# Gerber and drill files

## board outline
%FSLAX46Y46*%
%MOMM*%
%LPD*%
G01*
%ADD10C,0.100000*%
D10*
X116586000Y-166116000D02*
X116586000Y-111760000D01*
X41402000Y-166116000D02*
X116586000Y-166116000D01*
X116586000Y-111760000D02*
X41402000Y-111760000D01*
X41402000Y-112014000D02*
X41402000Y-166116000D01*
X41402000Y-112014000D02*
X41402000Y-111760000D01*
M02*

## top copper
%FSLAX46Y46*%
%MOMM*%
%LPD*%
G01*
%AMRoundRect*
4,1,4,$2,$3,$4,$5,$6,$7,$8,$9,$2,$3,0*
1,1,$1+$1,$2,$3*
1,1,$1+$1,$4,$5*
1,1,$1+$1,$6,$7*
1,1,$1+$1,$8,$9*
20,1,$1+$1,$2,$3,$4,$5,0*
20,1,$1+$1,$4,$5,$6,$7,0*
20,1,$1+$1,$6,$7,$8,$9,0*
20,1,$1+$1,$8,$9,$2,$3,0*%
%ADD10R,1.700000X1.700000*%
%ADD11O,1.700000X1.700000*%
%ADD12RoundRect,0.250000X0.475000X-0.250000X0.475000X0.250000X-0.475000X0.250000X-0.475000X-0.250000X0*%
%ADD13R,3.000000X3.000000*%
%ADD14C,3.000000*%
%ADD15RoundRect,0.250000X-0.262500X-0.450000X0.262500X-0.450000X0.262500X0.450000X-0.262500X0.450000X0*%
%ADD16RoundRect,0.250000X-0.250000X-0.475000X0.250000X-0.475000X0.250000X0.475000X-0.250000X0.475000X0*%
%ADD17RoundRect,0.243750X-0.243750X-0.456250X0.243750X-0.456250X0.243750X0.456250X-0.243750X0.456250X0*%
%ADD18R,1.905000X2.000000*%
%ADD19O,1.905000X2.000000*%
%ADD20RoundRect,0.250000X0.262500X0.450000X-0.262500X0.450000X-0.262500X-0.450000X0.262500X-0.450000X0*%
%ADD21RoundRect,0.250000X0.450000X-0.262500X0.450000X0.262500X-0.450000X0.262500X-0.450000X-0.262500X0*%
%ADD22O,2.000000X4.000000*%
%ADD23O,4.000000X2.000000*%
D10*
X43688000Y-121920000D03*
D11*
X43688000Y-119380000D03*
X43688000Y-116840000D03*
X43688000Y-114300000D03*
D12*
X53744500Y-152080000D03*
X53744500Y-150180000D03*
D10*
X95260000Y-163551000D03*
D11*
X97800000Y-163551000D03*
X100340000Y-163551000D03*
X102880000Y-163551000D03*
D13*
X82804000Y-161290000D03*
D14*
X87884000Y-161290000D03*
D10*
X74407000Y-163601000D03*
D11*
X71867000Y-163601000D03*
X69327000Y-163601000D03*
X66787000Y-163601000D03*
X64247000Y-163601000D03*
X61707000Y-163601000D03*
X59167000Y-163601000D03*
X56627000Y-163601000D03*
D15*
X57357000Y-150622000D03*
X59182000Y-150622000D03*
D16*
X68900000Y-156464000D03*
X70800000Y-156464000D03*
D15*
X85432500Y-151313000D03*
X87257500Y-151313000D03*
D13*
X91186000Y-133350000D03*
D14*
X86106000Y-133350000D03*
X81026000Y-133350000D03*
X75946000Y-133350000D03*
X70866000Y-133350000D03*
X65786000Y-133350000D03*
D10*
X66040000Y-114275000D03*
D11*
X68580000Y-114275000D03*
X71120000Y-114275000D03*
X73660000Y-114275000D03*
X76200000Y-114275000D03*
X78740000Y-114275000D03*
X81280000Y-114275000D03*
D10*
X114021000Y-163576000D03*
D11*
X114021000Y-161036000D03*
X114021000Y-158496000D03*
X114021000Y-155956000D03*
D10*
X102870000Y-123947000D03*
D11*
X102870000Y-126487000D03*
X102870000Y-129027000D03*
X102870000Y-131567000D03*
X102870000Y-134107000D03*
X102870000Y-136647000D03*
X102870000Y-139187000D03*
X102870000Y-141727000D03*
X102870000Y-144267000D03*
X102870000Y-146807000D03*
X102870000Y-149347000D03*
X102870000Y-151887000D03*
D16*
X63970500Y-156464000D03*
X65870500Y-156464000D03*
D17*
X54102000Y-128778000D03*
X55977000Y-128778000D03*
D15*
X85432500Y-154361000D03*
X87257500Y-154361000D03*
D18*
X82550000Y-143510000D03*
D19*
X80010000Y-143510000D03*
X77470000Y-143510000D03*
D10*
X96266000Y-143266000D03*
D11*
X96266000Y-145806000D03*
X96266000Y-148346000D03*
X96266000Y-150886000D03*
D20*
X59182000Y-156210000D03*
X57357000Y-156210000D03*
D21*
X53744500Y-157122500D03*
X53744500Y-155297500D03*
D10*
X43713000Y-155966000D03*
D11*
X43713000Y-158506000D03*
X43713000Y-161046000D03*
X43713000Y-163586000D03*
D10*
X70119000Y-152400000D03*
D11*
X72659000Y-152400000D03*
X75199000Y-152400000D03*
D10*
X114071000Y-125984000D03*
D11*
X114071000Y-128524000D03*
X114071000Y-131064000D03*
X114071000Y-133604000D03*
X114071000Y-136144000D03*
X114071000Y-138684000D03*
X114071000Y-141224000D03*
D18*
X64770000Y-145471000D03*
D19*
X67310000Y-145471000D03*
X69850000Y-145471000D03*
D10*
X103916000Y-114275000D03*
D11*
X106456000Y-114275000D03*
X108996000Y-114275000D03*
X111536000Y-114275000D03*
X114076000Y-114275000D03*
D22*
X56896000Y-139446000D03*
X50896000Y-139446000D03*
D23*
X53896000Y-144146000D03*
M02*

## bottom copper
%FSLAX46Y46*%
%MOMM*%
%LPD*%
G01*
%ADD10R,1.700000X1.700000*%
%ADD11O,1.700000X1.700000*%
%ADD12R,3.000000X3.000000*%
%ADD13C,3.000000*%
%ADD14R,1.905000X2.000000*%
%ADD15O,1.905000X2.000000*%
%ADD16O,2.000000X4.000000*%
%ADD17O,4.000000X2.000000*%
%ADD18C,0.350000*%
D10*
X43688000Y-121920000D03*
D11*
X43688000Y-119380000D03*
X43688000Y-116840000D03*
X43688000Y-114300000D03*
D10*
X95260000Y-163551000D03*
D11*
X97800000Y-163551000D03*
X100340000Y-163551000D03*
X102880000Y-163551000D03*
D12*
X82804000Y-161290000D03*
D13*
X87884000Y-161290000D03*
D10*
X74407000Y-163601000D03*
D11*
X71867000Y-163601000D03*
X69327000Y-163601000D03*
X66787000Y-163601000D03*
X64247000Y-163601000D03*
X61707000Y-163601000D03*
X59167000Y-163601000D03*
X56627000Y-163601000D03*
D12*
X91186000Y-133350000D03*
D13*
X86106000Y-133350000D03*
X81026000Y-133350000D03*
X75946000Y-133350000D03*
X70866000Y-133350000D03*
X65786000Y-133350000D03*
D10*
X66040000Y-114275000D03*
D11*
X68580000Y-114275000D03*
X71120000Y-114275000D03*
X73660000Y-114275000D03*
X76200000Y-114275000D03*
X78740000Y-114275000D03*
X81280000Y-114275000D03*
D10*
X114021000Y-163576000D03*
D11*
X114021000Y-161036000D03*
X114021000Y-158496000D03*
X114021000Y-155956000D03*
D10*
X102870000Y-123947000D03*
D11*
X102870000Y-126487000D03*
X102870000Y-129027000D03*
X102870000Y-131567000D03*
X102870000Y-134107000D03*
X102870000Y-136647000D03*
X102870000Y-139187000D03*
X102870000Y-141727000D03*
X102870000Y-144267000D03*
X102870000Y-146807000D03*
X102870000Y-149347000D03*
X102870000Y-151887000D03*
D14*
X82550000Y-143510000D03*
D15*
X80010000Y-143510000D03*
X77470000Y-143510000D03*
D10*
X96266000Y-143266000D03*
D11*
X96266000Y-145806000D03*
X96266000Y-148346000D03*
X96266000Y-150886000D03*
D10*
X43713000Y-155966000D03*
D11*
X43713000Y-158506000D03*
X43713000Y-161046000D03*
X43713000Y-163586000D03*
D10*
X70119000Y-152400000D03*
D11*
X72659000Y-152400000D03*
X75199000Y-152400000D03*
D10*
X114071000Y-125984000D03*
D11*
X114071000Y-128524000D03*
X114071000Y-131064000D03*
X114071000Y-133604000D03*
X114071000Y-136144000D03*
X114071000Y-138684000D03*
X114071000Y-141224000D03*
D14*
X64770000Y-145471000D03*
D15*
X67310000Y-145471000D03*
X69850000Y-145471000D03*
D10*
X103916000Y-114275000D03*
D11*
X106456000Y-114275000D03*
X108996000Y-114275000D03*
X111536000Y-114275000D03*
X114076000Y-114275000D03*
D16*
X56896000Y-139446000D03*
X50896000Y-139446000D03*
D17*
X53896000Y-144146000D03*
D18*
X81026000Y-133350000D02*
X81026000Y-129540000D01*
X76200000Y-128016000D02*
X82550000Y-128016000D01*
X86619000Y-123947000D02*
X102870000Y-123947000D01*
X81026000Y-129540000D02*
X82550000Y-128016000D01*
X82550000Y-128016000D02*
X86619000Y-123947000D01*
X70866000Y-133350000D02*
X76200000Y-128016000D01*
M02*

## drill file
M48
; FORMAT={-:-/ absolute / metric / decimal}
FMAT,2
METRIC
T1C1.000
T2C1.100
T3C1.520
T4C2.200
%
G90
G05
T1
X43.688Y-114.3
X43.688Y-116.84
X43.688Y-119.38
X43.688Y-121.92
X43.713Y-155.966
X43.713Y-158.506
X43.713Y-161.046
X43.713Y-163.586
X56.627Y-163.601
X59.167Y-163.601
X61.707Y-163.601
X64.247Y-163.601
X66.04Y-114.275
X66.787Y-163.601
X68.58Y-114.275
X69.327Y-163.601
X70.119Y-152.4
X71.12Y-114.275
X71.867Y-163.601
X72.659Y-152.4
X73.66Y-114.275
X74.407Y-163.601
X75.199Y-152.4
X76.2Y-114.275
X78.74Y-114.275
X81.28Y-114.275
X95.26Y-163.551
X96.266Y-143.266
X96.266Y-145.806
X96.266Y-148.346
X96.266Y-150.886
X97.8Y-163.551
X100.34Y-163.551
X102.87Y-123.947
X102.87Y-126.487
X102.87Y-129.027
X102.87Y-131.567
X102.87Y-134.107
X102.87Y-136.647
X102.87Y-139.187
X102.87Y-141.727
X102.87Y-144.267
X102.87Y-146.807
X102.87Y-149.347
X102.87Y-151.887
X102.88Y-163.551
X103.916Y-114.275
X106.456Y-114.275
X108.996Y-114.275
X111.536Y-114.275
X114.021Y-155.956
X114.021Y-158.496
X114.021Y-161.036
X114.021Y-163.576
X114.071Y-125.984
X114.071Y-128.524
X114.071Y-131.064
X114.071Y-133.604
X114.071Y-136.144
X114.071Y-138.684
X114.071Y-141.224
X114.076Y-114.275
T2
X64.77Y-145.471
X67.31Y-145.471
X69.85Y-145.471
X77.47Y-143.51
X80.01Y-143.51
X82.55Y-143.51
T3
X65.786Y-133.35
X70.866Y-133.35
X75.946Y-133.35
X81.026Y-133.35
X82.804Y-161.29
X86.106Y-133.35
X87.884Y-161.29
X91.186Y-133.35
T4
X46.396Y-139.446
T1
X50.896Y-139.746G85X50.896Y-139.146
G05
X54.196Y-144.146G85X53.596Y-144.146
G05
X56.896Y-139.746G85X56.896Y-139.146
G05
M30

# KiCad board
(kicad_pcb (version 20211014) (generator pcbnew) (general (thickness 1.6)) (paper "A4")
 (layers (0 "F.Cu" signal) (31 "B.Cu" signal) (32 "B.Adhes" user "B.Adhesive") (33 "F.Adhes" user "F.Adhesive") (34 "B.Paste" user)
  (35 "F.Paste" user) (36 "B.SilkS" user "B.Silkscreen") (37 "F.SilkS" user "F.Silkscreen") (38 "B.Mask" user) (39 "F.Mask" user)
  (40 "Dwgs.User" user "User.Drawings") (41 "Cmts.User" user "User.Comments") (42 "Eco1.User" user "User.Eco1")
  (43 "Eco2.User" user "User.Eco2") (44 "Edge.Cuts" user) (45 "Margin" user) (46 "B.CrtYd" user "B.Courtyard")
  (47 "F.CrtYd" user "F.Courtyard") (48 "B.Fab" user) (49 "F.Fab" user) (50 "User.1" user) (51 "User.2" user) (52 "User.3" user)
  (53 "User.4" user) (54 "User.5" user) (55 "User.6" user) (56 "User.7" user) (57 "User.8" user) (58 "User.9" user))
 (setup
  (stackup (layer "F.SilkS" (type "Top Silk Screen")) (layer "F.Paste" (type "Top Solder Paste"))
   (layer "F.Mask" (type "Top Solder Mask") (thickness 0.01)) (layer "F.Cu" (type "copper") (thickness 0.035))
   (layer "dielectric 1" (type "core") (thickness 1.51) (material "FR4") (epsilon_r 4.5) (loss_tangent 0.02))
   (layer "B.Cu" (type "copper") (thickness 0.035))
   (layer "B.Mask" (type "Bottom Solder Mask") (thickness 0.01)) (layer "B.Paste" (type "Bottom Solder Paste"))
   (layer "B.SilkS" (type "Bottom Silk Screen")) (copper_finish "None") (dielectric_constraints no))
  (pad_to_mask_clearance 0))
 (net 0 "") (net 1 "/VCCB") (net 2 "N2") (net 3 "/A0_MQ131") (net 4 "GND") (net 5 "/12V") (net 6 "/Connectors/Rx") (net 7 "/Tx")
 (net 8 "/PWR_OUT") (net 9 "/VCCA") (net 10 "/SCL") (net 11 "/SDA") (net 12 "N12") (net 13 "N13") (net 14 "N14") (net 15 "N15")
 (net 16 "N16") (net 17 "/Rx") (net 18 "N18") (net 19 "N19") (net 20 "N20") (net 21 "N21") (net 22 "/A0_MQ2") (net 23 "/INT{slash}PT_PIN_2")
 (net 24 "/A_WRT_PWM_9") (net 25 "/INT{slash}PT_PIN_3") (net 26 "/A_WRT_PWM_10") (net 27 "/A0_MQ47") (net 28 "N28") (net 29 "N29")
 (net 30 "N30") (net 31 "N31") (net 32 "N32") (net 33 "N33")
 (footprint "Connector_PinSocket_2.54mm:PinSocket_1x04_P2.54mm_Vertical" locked (layer "F.Cu") (at 43.688 121.92 180)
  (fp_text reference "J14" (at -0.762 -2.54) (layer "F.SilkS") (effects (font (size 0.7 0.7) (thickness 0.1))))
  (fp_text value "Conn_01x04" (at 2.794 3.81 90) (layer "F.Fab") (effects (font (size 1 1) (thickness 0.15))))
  (pad "1" thru_hole rect locked (at 0 0 180) (size 1.7 1.7) (drill 1) (layers *.Cu *.Mask) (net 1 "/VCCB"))
  (pad "2" thru_hole oval locked (at 0 2.54 180) (size 1.7 1.7) (drill 1) (layers *.Cu *.Mask) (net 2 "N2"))
  (pad "3" thru_hole oval locked (at 0 5.08 180) (size 1.7 1.7) (drill 1) (layers *.Cu *.Mask) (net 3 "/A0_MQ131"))
  (pad "4" thru_hole oval locked (at 0 7.62 180) (size 1.7 1.7) (drill 1) (layers *.Cu *.Mask) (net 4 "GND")))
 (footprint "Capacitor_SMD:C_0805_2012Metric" (layer "F.Cu") (at 53.7445 151.13 90)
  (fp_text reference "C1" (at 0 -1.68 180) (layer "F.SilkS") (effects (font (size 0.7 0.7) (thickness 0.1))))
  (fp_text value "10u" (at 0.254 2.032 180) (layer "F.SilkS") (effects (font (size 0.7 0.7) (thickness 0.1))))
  (pad "1" smd roundrect locked (at -0.95 0 90) (size 1 1.45) (layers "F.Cu" "F.Paste" "F.Mask") (roundrect_rratio 0.25) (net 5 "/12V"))
  (pad "2" smd roundrect locked (at 0.95 0 90) (size 1 1.45) (layers "F.Cu" "F.Paste" "F.Mask") (roundrect_rratio 0.25) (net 4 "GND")))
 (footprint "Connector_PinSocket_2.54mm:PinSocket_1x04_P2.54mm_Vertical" (layer "F.Cu") (at 95.26 163.551 90)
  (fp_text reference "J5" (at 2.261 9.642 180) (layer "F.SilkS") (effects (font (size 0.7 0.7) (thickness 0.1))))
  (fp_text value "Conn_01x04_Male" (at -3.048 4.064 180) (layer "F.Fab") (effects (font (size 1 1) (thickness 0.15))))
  (pad "1" thru_hole rect locked (at 0 0 90) (size 1.7 1.7) (drill 1) (layers *.Cu *.Mask) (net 1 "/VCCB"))
  (pad "2" thru_hole oval locked (at 0 2.54 90) (size 1.7 1.7) (drill 1) (layers *.Cu *.Mask) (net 4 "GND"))
  (pad "3" thru_hole oval locked (at 0 5.08 90) (size 1.7 1.7) (drill 1) (layers *.Cu *.Mask) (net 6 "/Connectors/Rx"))
  (pad "4" thru_hole oval locked (at 0 7.62 90) (size 1.7 1.7) (drill 1) (layers *.Cu *.Mask) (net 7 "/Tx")))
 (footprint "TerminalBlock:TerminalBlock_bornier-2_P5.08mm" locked (layer "F.Cu") (at 82.804 161.29)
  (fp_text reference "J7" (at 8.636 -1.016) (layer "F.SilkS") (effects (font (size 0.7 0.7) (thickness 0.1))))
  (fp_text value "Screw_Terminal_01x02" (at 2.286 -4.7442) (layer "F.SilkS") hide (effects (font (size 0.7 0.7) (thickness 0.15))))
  (pad "1" thru_hole rect locked (at 0 0) (size 3 3) (drill 1.52) (layers *.Cu *.Mask) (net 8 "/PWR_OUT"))
  (pad "2" thru_hole circle locked (at 5.08 0) (size 3 3) (drill 1.52) (layers *.Cu *.Mask) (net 4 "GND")))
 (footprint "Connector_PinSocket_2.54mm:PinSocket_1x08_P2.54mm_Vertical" (layer "F.Cu") (at 74.407 163.601 -90)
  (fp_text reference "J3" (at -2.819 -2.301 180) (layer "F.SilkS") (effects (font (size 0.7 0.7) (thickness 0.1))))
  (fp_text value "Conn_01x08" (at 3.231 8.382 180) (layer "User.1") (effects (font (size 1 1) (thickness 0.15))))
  (pad "1" thru_hole rect locked (at 0 0 270) (size 1.7 1.7) (drill 1) (layers *.Cu *.Mask) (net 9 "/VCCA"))
  (pad "2" thru_hole oval locked (at 0 2.54 270) (size 1.7 1.7) (drill 1) (layers *.Cu *.Mask) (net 4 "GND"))
  (pad "3" thru_hole oval locked (at 0 5.08 270) (size 1.7 1.7) (drill 1) (layers *.Cu *.Mask) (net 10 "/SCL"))
  (pad "4" thru_hole oval locked (at 0 7.62 270) (size 1.7 1.7) (drill 1) (layers *.Cu *.Mask) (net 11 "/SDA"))
  (pad "5" thru_hole oval locked (at 0 10.16 270) (size 1.7 1.7) (drill 1) (layers *.Cu *.Mask) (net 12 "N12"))
  (pad "6" thru_hole oval locked (at 0 12.7 270) (size 1.7 1.7) (drill 1) (layers *.Cu *.Mask) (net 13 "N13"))
  (pad "7" thru_hole oval locked (at 0 15.24 270) (size 1.7 1.7) (drill 1) (layers *.Cu *.Mask) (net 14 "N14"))
  (pad "8" thru_hole oval locked (at 0 17.78 270) (size 1.7 1.7) (drill 1) (layers *.Cu *.Mask) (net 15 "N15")))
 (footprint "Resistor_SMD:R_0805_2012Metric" (layer "F.Cu") (at 58.2695 150.622)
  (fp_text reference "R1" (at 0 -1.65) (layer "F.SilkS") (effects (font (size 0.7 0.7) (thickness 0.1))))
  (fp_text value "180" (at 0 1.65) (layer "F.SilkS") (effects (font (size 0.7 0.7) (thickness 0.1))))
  (pad "1" smd roundrect locked (at -0.9125 0) (size 1.025 1.4) (layers "F.Cu" "F.Paste" "F.Mask") (roundrect_rratio 0.243902)
   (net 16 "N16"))
  (pad "2" smd roundrect locked (at 0.9125 0) (size 1.025 1.4) (layers "F.Cu" "F.Paste" "F.Mask") (roundrect_rratio 0.243902)
   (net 1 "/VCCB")))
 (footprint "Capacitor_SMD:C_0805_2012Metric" (layer "F.Cu") (at 69.85 156.464)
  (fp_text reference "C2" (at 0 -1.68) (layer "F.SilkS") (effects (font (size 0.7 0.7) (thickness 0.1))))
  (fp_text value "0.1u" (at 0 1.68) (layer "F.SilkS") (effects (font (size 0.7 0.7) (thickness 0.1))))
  (pad "1" smd roundrect locked (at -0.95 0) (size 1 1.45) (layers "F.Cu" "F.Paste" "F.Mask") (roundrect_rratio 0.25) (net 9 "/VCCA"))
  (pad "2" smd roundrect locked (at 0.95 0) (size 1 1.45) (layers "F.Cu" "F.Paste" "F.Mask") (roundrect_rratio 0.25) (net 4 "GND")))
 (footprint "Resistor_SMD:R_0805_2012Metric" (layer "F.Cu") (at 86.345 151.313)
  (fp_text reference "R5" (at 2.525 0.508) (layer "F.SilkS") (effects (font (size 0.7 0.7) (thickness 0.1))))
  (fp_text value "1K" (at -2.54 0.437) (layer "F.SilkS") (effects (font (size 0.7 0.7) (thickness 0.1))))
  (pad "1" smd roundrect locked (at -0.9125 0) (size 1.025 1.4) (layers "F.Cu" "F.Paste" "F.Mask") (roundrect_rratio 0.243902)
   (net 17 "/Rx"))
  (pad "2" smd roundrect locked (at 0.9125 0) (size 1.025 1.4) (layers "F.Cu" "F.Paste" "F.Mask") (roundrect_rratio 0.243902)
   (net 6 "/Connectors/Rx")))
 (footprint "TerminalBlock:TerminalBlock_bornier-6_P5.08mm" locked (layer "F.Cu") (at 91.186 133.35 180)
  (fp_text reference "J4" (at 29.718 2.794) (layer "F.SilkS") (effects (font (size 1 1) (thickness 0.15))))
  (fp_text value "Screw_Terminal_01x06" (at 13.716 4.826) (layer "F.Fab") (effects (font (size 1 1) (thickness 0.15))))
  (pad "1" thru_hole rect locked (at 0 0 180) (size 3 3) (drill 1.52) (layers *.Cu *.Mask) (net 4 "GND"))
  (pad "2" thru_hole circle locked (at 5.08 0 180) (size 3 3) (drill 1.52) (layers *.Cu *.Mask) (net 5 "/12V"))
  (pad "3" thru_hole circle locked (at 10.16 0 180) (size 3 3) (drill 1.52) (layers *.Cu *.Mask) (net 4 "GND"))
  (pad "4" thru_hole circle locked (at 15.24 0 180) (size 3 3) (drill 1.52) (layers *.Cu *.Mask) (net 5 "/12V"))
  (pad "5" thru_hole circle locked (at 20.32 0 180) (size 3 3) (drill 1.52) (layers *.Cu *.Mask) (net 4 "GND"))
  (pad "6" thru_hole circle locked (at 25.4 0 180) (size 3 3) (drill 1.52) (layers *.Cu *.Mask) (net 5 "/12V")))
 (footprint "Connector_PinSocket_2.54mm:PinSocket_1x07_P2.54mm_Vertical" (layer "F.Cu") (at 66.04 114.275 90)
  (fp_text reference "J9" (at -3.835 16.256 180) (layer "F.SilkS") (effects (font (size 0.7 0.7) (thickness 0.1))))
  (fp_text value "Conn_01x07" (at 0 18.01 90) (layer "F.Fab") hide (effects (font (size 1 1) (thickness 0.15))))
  (pad "1" thru_hole rect locked (at 0 0 90) (size 1.7 1.7) (drill 1) (layers *.Cu *.Mask) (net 9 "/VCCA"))
  (pad "2" thru_hole oval locked (at 0 2.54 90) (size 1.7 1.7) (drill 1) (layers *.Cu *.Mask) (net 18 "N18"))
  (pad "3" thru_hole oval locked (at 0 5.08 90) (size 1.7 1.7) (drill 1) (layers *.Cu *.Mask) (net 4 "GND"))
  (pad "4" thru_hole oval locked (at 0 7.62 90) (size 1.7 1.7) (drill 1) (layers *.Cu *.Mask) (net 10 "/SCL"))
  (pad "5" thru_hole oval locked (at 0 10.16 90) (size 1.7 1.7) (drill 1) (layers *.Cu *.Mask) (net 11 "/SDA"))
  (pad "6" thru_hole oval locked (at 0 12.7 90) (size 1.7 1.7) (drill 1) (layers *.Cu *.Mask) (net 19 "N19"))
  (pad "7" thru_hole oval locked (at 0 15.24 90) (size 1.7 1.7) (drill 1) (layers *.Cu *.Mask) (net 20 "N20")))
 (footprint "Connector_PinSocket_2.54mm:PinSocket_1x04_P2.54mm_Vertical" (layer "F.Cu") (at 114.021 163.576 180)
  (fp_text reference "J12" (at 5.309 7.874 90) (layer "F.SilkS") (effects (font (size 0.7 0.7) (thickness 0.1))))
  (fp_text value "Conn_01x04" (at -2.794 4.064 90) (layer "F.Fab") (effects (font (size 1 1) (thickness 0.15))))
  (pad "1" thru_hole rect locked (at 0 0 180) (size 1.7 1.7) (drill 1) (layers *.Cu *.Mask) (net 1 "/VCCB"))
  (pad "2" thru_hole oval locked (at 0 2.54 180) (size 1.7 1.7) (drill 1) (layers *.Cu *.Mask) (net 4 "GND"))
  (pad "3" thru_hole oval locked (at 0 5.08 180) (size 1.7 1.7) (drill 1) (layers *.Cu *.Mask) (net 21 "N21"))
  (pad "4" thru_hole oval locked (at 0 7.62 180) (size 1.7 1.7) (drill 1) (layers *.Cu *.Mask) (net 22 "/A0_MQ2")))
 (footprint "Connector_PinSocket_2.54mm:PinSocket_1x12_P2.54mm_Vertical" (layer "F.Cu") (at 102.87 123.947)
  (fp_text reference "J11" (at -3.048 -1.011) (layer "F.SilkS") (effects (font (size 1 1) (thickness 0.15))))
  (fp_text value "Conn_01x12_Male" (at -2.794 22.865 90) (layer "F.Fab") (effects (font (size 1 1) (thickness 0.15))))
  (pad "1" thru_hole rect locked (at 0 0) (size 1.7 1.7) (drill 1) (layers *.Cu *.Mask) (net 4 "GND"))
  (pad "2" thru_hole oval locked (at 0 2.54) (size 1.7 1.7) (drill 1) (layers *.Cu *.Mask) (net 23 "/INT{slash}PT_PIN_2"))
  (pad "3" thru_hole oval locked (at 0 5.08) (size 1.7 1.7) (drill 1) (layers *.Cu *.Mask) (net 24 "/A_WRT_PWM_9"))
  (pad "4" thru_hole oval locked (at 0 7.62) (size 1.7 1.7) (drill 1) (layers *.Cu *.Mask) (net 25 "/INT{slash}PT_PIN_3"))
  (pad "5" thru_hole oval locked (at 0 10.16) (size 1.7 1.7) (drill 1) (layers *.Cu *.Mask) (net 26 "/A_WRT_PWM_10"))
  (pad "6" thru_hole oval locked (at 0 12.7) (size 1.7 1.7) (drill 1) (layers *.Cu *.Mask) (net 11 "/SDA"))
  (pad "7" thru_hole oval locked (at 0 15.24) (size 1.7 1.7) (drill 1) (layers *.Cu *.Mask) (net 10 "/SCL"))
  (pad "8" thru_hole oval locked (at 0 17.78) (size 1.7 1.7) (drill 1) (layers *.Cu *.Mask) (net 22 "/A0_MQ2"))
  (pad "9" thru_hole oval locked (at 0 20.32) (size 1.7 1.7) (drill 1) (layers *.Cu *.Mask) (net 3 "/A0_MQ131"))
  (pad "10" thru_hole oval locked (at 0 22.86) (size 1.7 1.7) (drill 1) (layers *.Cu *.Mask) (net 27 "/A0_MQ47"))
  (pad "11" thru_hole oval locked (at 0 25.4) (size 1.7 1.7) (drill 1) (layers *.Cu *.Mask) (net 7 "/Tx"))
  (pad "12" thru_hole oval locked (at 0 27.94) (size 1.7 1.7) (drill 1) (layers *.Cu *.Mask) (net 17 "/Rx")))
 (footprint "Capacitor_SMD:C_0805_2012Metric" (layer "F.Cu") (at 64.9205 156.464)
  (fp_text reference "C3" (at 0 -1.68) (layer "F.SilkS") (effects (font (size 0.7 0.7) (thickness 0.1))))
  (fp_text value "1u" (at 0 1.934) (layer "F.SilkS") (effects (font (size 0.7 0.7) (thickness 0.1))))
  (pad "1" smd roundrect locked (at -0.95 0) (size 1 1.45) (layers "F.Cu" "F.Paste" "F.Mask") (roundrect_rratio 0.25) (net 1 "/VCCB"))
  (pad "2" smd roundrect locked (at 0.95 0) (size 1 1.45) (layers "F.Cu" "F.Paste" "F.Mask") (roundrect_rratio 0.25) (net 4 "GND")))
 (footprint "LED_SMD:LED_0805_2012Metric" (layer "F.Cu") (at 55.0395 128.778)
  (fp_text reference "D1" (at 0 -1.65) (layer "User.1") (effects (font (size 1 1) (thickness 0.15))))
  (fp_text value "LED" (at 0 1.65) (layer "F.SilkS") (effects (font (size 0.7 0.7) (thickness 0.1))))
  (pad "1" smd roundrect locked (at -0.9375 0) (size 0.975 1.4) (layers "F.Cu" "F.Paste" "F.Mask") (roundrect_rratio 0.25) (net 4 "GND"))
  (pad "2" smd roundrect locked (at 0.9375 0) (size 0.975 1.4) (layers "F.Cu" "F.Paste" "F.Mask") (roundrect_rratio 0.25) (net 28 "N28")))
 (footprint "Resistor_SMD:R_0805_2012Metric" (layer "F.Cu") (at 86.345 154.361)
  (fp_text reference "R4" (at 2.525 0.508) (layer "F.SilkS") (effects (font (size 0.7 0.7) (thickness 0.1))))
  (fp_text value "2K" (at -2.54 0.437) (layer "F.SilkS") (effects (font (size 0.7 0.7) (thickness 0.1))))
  (pad "1" smd roundrect locked (at -0.9125 0) (size 1.025 1.4) (layers "F.Cu" "F.Paste" "F.Mask") (roundrect_rratio 0.243902) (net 4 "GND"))
  (pad "2" smd roundrect locked (at 0.9125 0) (size 1.025 1.4) (layers "F.Cu" "F.Paste" "F.Mask") (roundrect_rratio 0.243902)
   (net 6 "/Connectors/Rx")))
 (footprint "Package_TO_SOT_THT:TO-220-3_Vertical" (layer "F.Cu") (at 82.55 143.51 180)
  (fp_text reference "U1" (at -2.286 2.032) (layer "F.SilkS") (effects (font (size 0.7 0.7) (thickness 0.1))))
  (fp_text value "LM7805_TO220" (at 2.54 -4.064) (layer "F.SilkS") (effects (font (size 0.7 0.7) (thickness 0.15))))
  (pad "1" thru_hole rect locked (at 0 0 180) (size 1.905 2) (drill 1.1) (layers *.Cu *.Mask) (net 5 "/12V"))
  (pad "2" thru_hole oval locked (at 2.54 0 180) (size 1.905 2) (drill 1.1) (layers *.Cu *.Mask) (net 4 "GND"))
  (pad "3" thru_hole oval locked (at 5.08 0 180) (size 1.905 2) (drill 1.1) (layers *.Cu *.Mask) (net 9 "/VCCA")))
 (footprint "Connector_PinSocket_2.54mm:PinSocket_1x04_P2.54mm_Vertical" (layer "F.Cu") (at 96.266 143.266)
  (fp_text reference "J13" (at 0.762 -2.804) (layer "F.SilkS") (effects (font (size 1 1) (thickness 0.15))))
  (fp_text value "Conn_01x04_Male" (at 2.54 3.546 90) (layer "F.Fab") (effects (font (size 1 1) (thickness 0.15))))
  (pad "1" thru_hole rect locked (at 0 0) (size 1.7 1.7) (drill 1) (layers *.Cu *.Mask) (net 23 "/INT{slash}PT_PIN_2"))
  (pad "2" thru_hole oval locked (at 0 2.54) (size 1.7 1.7) (drill 1) (layers *.Cu *.Mask) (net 24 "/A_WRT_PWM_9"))
  (pad "3" thru_hole oval locked (at 0 5.08) (size 1.7 1.7) (drill 1) (layers *.Cu *.Mask) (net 25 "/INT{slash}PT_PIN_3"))
  (pad "4" thru_hole oval locked (at 0 7.62) (size 1.7 1.7) (drill 1) (layers *.Cu *.Mask) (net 26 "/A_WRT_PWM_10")))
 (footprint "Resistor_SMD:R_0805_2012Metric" (layer "F.Cu") (at 58.2695 156.21 180)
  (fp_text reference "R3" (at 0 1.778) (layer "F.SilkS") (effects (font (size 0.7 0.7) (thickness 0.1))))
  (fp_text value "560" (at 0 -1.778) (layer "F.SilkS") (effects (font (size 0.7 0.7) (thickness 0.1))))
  (pad "1" smd roundrect locked (at -0.9125 0 180) (size 1.025 1.4) (layers "F.Cu" "F.Paste" "F.Mask") (roundrect_rratio 0.243902)
   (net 4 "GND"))
  (pad "2" smd roundrect locked (at 0.9125 0 180) (size 1.025 1.4) (layers "F.Cu" "F.Paste" "F.Mask") (roundrect_rratio 0.243902)
   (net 16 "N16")))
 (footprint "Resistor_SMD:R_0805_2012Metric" (layer "F.Cu") (at 53.7445 156.21 90)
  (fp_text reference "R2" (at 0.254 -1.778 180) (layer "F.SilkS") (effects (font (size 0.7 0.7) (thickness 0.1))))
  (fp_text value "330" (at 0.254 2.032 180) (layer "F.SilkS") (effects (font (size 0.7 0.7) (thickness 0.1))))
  (pad "1" smd roundrect locked (at -0.9125 0 90) (size 1.025 1.4) (layers "F.Cu" "F.Paste" "F.Mask") (roundrect_rratio 0.243902)
   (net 28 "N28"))
  (pad "2" smd roundrect locked (at 0.9125 0 90) (size 1.025 1.4) (layers "F.Cu" "F.Paste" "F.Mask") (roundrect_rratio 0.243902)
   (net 5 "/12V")))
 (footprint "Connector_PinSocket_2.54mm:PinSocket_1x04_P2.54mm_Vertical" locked (layer "F.Cu") (at 43.713 155.966)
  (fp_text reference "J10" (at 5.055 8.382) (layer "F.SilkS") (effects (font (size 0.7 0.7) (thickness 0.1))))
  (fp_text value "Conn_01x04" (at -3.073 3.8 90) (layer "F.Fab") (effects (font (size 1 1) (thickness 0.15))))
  (pad "1" thru_hole rect locked (at 0 0) (size 1.7 1.7) (drill 1) (layers *.Cu *.Mask) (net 1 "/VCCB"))
  (pad "2" thru_hole oval locked (at 0 2.54) (size 1.7 1.7) (drill 1) (layers *.Cu *.Mask) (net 4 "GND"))
  (pad "3" thru_hole oval locked (at 0 5.08) (size 1.7 1.7) (drill 1) (layers *.Cu *.Mask) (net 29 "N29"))
  (pad "4" thru_hole oval locked (at 0 7.62) (size 1.7 1.7) (drill 1) (layers *.Cu *.Mask) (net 27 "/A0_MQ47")))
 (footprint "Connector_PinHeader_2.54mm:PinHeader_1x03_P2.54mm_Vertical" (layer "F.Cu") (at 70.119 152.4 90)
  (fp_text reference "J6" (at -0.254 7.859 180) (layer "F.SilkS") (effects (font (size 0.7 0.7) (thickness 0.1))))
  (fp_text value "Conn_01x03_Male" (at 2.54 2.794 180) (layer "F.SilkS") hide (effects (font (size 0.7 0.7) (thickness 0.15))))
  (pad "1" thru_hole rect locked (at 0 0 90) (size 1.7 1.7) (drill 1) (layers *.Cu *.Mask) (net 1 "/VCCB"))
  (pad "2" thru_hole oval locked (at 0 2.54 90) (size 1.7 1.7) (drill 1) (layers *.Cu *.Mask) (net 8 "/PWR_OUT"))
  (pad "3" thru_hole oval locked (at 0 5.08 90) (size 1.7 1.7) (drill 1) (layers *.Cu *.Mask) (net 9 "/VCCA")))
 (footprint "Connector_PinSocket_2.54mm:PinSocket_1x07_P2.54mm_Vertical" (layer "F.Cu") (at 114.071 125.984)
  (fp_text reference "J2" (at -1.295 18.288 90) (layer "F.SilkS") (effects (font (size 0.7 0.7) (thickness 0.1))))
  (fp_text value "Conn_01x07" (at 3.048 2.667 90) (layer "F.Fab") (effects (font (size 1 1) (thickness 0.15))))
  (pad "1" thru_hole rect locked (at 0 0) (size 1.7 1.7) (drill 1) (layers *.Cu *.Mask) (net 9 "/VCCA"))
  (pad "2" thru_hole oval locked (at 0 2.54) (size 1.7 1.7) (drill 1) (layers *.Cu *.Mask) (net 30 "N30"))
  (pad "3" thru_hole oval locked (at 0 5.08) (size 1.7 1.7) (drill 1) (layers *.Cu *.Mask) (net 4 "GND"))
  (pad "4" thru_hole oval locked (at 0 7.62) (size 1.7 1.7) (drill 1) (layers *.Cu *.Mask) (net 10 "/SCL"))
  (pad "5" thru_hole oval locked (at 0 10.16) (size 1.7 1.7) (drill 1) (layers *.Cu *.Mask) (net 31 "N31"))
  (pad "6" thru_hole oval locked (at 0 12.7) (size 1.7 1.7) (drill 1) (layers *.Cu *.Mask) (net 11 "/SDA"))
  (pad "7" thru_hole oval locked (at 0 15.24) (size 1.7 1.7) (drill 1) (layers *.Cu *.Mask) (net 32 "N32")))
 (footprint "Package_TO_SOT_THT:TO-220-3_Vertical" (layer "F.Cu") (at 64.77 145.471)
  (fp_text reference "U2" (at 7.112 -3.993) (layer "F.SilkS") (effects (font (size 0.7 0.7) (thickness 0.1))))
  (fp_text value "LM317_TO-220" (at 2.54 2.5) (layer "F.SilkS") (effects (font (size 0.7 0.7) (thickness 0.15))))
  (pad "1" thru_hole rect locked (at 0 0) (size 1.905 2) (drill 1.1) (layers *.Cu *.Mask) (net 16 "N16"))
  (pad "2" thru_hole oval locked (at 2.54 0) (size 1.905 2) (drill 1.1) (layers *.Cu *.Mask) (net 1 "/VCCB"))
  (pad "3" thru_hole oval locked (at 5.08 0) (size 1.905 2) (drill 1.1) (layers *.Cu *.Mask) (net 5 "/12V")))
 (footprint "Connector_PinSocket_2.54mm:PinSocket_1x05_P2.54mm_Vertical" (layer "F.Cu") (at 103.916 114.275 90)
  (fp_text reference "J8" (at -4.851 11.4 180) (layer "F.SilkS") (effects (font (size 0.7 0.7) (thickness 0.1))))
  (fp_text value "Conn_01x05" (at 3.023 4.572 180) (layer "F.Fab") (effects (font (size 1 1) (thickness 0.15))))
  (pad "1" thru_hole rect locked (at 0 0 90) (size 1.7 1.7) (drill 1) (layers *.Cu *.Mask) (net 9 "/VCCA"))
  (pad "2" thru_hole oval locked (at 0 2.54 90) (size 1.7 1.7) (drill 1) (layers *.Cu *.Mask) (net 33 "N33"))
  (pad "3" thru_hole oval locked (at 0 5.08 90) (size 1.7 1.7) (drill 1) (layers *.Cu *.Mask) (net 4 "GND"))
  (pad "4" thru_hole oval locked (at 0 7.62 90) (size 1.7 1.7) (drill 1) (layers *.Cu *.Mask) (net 10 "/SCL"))
  (pad "5" thru_hole oval locked (at 0 10.16 90) (size 1.7 1.7) (drill 1) (layers *.Cu *.Mask) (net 11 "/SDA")))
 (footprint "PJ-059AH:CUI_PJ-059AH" (layer "F.Cu") (at 56.896 139.446 180)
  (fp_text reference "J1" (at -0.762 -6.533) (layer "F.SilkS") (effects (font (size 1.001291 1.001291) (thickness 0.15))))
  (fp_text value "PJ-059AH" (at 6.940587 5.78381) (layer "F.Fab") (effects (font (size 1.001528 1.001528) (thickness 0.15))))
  (pad "" np_thru_hole circle locked (at 10.5 0 180) (size 2.2 2.2) (drill 2.2) (layers *.Cu *.Mask))
  (pad "1" thru_hole oval locked (at 0 0 180) (size 2 4) (drill oval 1 1.6) (layers *.Cu *.Mask) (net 5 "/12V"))
  (pad "2" thru_hole oval locked (at 6 0 180) (size 2 4) (drill oval 1 1.6) (layers *.Cu *.Mask) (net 4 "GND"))
  (pad "3" thru_hole oval locked (at 3 -4.7 180) (size 4 2) (drill oval 1.6 1) (layers *.Cu *.Mask) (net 4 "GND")))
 (gr_line (start 116.586 166.116) (end 116.586 111.76) (layer "Edge.Cuts") (width 0.1))
 (gr_line (start 41.402 166.116) (end 116.586 166.116) (layer "Edge.Cuts") (width 0.1))
 (gr_line (start 116.586 111.76) (end 41.402 111.76) (layer "Edge.Cuts") (width 0.1))
 (gr_line (start 41.402 112.014) (end 41.402 166.116) (layer "Edge.Cuts") (width 0.1))
 (gr_line (start 41.402 112.014) (end 41.402 111.76) (layer "Edge.Cuts") (width 0.1))
 (segment (start 81.026 133.35) (end 81.026 129.54) (width 0.35) (layer "B.Cu") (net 4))
 (segment (start 76.2 128.016) (end 82.55 128.016) (width 0.35) (layer "B.Cu") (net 4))
 (segment (start 86.619 123.947) (end 102.87 123.947) (width 0.35) (layer "B.Cu") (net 4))
 (segment (start 81.026 129.54) (end 82.55 128.016) (width 0.35) (layer "B.Cu") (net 4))
 (segment (start 82.55 128.016) (end 86.619 123.947) (width 0.35) (layer "B.Cu") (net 4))
 (segment (start 70.866 133.35) (end 76.2 128.016) (width 0.35) (layer "B.Cu") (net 4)))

